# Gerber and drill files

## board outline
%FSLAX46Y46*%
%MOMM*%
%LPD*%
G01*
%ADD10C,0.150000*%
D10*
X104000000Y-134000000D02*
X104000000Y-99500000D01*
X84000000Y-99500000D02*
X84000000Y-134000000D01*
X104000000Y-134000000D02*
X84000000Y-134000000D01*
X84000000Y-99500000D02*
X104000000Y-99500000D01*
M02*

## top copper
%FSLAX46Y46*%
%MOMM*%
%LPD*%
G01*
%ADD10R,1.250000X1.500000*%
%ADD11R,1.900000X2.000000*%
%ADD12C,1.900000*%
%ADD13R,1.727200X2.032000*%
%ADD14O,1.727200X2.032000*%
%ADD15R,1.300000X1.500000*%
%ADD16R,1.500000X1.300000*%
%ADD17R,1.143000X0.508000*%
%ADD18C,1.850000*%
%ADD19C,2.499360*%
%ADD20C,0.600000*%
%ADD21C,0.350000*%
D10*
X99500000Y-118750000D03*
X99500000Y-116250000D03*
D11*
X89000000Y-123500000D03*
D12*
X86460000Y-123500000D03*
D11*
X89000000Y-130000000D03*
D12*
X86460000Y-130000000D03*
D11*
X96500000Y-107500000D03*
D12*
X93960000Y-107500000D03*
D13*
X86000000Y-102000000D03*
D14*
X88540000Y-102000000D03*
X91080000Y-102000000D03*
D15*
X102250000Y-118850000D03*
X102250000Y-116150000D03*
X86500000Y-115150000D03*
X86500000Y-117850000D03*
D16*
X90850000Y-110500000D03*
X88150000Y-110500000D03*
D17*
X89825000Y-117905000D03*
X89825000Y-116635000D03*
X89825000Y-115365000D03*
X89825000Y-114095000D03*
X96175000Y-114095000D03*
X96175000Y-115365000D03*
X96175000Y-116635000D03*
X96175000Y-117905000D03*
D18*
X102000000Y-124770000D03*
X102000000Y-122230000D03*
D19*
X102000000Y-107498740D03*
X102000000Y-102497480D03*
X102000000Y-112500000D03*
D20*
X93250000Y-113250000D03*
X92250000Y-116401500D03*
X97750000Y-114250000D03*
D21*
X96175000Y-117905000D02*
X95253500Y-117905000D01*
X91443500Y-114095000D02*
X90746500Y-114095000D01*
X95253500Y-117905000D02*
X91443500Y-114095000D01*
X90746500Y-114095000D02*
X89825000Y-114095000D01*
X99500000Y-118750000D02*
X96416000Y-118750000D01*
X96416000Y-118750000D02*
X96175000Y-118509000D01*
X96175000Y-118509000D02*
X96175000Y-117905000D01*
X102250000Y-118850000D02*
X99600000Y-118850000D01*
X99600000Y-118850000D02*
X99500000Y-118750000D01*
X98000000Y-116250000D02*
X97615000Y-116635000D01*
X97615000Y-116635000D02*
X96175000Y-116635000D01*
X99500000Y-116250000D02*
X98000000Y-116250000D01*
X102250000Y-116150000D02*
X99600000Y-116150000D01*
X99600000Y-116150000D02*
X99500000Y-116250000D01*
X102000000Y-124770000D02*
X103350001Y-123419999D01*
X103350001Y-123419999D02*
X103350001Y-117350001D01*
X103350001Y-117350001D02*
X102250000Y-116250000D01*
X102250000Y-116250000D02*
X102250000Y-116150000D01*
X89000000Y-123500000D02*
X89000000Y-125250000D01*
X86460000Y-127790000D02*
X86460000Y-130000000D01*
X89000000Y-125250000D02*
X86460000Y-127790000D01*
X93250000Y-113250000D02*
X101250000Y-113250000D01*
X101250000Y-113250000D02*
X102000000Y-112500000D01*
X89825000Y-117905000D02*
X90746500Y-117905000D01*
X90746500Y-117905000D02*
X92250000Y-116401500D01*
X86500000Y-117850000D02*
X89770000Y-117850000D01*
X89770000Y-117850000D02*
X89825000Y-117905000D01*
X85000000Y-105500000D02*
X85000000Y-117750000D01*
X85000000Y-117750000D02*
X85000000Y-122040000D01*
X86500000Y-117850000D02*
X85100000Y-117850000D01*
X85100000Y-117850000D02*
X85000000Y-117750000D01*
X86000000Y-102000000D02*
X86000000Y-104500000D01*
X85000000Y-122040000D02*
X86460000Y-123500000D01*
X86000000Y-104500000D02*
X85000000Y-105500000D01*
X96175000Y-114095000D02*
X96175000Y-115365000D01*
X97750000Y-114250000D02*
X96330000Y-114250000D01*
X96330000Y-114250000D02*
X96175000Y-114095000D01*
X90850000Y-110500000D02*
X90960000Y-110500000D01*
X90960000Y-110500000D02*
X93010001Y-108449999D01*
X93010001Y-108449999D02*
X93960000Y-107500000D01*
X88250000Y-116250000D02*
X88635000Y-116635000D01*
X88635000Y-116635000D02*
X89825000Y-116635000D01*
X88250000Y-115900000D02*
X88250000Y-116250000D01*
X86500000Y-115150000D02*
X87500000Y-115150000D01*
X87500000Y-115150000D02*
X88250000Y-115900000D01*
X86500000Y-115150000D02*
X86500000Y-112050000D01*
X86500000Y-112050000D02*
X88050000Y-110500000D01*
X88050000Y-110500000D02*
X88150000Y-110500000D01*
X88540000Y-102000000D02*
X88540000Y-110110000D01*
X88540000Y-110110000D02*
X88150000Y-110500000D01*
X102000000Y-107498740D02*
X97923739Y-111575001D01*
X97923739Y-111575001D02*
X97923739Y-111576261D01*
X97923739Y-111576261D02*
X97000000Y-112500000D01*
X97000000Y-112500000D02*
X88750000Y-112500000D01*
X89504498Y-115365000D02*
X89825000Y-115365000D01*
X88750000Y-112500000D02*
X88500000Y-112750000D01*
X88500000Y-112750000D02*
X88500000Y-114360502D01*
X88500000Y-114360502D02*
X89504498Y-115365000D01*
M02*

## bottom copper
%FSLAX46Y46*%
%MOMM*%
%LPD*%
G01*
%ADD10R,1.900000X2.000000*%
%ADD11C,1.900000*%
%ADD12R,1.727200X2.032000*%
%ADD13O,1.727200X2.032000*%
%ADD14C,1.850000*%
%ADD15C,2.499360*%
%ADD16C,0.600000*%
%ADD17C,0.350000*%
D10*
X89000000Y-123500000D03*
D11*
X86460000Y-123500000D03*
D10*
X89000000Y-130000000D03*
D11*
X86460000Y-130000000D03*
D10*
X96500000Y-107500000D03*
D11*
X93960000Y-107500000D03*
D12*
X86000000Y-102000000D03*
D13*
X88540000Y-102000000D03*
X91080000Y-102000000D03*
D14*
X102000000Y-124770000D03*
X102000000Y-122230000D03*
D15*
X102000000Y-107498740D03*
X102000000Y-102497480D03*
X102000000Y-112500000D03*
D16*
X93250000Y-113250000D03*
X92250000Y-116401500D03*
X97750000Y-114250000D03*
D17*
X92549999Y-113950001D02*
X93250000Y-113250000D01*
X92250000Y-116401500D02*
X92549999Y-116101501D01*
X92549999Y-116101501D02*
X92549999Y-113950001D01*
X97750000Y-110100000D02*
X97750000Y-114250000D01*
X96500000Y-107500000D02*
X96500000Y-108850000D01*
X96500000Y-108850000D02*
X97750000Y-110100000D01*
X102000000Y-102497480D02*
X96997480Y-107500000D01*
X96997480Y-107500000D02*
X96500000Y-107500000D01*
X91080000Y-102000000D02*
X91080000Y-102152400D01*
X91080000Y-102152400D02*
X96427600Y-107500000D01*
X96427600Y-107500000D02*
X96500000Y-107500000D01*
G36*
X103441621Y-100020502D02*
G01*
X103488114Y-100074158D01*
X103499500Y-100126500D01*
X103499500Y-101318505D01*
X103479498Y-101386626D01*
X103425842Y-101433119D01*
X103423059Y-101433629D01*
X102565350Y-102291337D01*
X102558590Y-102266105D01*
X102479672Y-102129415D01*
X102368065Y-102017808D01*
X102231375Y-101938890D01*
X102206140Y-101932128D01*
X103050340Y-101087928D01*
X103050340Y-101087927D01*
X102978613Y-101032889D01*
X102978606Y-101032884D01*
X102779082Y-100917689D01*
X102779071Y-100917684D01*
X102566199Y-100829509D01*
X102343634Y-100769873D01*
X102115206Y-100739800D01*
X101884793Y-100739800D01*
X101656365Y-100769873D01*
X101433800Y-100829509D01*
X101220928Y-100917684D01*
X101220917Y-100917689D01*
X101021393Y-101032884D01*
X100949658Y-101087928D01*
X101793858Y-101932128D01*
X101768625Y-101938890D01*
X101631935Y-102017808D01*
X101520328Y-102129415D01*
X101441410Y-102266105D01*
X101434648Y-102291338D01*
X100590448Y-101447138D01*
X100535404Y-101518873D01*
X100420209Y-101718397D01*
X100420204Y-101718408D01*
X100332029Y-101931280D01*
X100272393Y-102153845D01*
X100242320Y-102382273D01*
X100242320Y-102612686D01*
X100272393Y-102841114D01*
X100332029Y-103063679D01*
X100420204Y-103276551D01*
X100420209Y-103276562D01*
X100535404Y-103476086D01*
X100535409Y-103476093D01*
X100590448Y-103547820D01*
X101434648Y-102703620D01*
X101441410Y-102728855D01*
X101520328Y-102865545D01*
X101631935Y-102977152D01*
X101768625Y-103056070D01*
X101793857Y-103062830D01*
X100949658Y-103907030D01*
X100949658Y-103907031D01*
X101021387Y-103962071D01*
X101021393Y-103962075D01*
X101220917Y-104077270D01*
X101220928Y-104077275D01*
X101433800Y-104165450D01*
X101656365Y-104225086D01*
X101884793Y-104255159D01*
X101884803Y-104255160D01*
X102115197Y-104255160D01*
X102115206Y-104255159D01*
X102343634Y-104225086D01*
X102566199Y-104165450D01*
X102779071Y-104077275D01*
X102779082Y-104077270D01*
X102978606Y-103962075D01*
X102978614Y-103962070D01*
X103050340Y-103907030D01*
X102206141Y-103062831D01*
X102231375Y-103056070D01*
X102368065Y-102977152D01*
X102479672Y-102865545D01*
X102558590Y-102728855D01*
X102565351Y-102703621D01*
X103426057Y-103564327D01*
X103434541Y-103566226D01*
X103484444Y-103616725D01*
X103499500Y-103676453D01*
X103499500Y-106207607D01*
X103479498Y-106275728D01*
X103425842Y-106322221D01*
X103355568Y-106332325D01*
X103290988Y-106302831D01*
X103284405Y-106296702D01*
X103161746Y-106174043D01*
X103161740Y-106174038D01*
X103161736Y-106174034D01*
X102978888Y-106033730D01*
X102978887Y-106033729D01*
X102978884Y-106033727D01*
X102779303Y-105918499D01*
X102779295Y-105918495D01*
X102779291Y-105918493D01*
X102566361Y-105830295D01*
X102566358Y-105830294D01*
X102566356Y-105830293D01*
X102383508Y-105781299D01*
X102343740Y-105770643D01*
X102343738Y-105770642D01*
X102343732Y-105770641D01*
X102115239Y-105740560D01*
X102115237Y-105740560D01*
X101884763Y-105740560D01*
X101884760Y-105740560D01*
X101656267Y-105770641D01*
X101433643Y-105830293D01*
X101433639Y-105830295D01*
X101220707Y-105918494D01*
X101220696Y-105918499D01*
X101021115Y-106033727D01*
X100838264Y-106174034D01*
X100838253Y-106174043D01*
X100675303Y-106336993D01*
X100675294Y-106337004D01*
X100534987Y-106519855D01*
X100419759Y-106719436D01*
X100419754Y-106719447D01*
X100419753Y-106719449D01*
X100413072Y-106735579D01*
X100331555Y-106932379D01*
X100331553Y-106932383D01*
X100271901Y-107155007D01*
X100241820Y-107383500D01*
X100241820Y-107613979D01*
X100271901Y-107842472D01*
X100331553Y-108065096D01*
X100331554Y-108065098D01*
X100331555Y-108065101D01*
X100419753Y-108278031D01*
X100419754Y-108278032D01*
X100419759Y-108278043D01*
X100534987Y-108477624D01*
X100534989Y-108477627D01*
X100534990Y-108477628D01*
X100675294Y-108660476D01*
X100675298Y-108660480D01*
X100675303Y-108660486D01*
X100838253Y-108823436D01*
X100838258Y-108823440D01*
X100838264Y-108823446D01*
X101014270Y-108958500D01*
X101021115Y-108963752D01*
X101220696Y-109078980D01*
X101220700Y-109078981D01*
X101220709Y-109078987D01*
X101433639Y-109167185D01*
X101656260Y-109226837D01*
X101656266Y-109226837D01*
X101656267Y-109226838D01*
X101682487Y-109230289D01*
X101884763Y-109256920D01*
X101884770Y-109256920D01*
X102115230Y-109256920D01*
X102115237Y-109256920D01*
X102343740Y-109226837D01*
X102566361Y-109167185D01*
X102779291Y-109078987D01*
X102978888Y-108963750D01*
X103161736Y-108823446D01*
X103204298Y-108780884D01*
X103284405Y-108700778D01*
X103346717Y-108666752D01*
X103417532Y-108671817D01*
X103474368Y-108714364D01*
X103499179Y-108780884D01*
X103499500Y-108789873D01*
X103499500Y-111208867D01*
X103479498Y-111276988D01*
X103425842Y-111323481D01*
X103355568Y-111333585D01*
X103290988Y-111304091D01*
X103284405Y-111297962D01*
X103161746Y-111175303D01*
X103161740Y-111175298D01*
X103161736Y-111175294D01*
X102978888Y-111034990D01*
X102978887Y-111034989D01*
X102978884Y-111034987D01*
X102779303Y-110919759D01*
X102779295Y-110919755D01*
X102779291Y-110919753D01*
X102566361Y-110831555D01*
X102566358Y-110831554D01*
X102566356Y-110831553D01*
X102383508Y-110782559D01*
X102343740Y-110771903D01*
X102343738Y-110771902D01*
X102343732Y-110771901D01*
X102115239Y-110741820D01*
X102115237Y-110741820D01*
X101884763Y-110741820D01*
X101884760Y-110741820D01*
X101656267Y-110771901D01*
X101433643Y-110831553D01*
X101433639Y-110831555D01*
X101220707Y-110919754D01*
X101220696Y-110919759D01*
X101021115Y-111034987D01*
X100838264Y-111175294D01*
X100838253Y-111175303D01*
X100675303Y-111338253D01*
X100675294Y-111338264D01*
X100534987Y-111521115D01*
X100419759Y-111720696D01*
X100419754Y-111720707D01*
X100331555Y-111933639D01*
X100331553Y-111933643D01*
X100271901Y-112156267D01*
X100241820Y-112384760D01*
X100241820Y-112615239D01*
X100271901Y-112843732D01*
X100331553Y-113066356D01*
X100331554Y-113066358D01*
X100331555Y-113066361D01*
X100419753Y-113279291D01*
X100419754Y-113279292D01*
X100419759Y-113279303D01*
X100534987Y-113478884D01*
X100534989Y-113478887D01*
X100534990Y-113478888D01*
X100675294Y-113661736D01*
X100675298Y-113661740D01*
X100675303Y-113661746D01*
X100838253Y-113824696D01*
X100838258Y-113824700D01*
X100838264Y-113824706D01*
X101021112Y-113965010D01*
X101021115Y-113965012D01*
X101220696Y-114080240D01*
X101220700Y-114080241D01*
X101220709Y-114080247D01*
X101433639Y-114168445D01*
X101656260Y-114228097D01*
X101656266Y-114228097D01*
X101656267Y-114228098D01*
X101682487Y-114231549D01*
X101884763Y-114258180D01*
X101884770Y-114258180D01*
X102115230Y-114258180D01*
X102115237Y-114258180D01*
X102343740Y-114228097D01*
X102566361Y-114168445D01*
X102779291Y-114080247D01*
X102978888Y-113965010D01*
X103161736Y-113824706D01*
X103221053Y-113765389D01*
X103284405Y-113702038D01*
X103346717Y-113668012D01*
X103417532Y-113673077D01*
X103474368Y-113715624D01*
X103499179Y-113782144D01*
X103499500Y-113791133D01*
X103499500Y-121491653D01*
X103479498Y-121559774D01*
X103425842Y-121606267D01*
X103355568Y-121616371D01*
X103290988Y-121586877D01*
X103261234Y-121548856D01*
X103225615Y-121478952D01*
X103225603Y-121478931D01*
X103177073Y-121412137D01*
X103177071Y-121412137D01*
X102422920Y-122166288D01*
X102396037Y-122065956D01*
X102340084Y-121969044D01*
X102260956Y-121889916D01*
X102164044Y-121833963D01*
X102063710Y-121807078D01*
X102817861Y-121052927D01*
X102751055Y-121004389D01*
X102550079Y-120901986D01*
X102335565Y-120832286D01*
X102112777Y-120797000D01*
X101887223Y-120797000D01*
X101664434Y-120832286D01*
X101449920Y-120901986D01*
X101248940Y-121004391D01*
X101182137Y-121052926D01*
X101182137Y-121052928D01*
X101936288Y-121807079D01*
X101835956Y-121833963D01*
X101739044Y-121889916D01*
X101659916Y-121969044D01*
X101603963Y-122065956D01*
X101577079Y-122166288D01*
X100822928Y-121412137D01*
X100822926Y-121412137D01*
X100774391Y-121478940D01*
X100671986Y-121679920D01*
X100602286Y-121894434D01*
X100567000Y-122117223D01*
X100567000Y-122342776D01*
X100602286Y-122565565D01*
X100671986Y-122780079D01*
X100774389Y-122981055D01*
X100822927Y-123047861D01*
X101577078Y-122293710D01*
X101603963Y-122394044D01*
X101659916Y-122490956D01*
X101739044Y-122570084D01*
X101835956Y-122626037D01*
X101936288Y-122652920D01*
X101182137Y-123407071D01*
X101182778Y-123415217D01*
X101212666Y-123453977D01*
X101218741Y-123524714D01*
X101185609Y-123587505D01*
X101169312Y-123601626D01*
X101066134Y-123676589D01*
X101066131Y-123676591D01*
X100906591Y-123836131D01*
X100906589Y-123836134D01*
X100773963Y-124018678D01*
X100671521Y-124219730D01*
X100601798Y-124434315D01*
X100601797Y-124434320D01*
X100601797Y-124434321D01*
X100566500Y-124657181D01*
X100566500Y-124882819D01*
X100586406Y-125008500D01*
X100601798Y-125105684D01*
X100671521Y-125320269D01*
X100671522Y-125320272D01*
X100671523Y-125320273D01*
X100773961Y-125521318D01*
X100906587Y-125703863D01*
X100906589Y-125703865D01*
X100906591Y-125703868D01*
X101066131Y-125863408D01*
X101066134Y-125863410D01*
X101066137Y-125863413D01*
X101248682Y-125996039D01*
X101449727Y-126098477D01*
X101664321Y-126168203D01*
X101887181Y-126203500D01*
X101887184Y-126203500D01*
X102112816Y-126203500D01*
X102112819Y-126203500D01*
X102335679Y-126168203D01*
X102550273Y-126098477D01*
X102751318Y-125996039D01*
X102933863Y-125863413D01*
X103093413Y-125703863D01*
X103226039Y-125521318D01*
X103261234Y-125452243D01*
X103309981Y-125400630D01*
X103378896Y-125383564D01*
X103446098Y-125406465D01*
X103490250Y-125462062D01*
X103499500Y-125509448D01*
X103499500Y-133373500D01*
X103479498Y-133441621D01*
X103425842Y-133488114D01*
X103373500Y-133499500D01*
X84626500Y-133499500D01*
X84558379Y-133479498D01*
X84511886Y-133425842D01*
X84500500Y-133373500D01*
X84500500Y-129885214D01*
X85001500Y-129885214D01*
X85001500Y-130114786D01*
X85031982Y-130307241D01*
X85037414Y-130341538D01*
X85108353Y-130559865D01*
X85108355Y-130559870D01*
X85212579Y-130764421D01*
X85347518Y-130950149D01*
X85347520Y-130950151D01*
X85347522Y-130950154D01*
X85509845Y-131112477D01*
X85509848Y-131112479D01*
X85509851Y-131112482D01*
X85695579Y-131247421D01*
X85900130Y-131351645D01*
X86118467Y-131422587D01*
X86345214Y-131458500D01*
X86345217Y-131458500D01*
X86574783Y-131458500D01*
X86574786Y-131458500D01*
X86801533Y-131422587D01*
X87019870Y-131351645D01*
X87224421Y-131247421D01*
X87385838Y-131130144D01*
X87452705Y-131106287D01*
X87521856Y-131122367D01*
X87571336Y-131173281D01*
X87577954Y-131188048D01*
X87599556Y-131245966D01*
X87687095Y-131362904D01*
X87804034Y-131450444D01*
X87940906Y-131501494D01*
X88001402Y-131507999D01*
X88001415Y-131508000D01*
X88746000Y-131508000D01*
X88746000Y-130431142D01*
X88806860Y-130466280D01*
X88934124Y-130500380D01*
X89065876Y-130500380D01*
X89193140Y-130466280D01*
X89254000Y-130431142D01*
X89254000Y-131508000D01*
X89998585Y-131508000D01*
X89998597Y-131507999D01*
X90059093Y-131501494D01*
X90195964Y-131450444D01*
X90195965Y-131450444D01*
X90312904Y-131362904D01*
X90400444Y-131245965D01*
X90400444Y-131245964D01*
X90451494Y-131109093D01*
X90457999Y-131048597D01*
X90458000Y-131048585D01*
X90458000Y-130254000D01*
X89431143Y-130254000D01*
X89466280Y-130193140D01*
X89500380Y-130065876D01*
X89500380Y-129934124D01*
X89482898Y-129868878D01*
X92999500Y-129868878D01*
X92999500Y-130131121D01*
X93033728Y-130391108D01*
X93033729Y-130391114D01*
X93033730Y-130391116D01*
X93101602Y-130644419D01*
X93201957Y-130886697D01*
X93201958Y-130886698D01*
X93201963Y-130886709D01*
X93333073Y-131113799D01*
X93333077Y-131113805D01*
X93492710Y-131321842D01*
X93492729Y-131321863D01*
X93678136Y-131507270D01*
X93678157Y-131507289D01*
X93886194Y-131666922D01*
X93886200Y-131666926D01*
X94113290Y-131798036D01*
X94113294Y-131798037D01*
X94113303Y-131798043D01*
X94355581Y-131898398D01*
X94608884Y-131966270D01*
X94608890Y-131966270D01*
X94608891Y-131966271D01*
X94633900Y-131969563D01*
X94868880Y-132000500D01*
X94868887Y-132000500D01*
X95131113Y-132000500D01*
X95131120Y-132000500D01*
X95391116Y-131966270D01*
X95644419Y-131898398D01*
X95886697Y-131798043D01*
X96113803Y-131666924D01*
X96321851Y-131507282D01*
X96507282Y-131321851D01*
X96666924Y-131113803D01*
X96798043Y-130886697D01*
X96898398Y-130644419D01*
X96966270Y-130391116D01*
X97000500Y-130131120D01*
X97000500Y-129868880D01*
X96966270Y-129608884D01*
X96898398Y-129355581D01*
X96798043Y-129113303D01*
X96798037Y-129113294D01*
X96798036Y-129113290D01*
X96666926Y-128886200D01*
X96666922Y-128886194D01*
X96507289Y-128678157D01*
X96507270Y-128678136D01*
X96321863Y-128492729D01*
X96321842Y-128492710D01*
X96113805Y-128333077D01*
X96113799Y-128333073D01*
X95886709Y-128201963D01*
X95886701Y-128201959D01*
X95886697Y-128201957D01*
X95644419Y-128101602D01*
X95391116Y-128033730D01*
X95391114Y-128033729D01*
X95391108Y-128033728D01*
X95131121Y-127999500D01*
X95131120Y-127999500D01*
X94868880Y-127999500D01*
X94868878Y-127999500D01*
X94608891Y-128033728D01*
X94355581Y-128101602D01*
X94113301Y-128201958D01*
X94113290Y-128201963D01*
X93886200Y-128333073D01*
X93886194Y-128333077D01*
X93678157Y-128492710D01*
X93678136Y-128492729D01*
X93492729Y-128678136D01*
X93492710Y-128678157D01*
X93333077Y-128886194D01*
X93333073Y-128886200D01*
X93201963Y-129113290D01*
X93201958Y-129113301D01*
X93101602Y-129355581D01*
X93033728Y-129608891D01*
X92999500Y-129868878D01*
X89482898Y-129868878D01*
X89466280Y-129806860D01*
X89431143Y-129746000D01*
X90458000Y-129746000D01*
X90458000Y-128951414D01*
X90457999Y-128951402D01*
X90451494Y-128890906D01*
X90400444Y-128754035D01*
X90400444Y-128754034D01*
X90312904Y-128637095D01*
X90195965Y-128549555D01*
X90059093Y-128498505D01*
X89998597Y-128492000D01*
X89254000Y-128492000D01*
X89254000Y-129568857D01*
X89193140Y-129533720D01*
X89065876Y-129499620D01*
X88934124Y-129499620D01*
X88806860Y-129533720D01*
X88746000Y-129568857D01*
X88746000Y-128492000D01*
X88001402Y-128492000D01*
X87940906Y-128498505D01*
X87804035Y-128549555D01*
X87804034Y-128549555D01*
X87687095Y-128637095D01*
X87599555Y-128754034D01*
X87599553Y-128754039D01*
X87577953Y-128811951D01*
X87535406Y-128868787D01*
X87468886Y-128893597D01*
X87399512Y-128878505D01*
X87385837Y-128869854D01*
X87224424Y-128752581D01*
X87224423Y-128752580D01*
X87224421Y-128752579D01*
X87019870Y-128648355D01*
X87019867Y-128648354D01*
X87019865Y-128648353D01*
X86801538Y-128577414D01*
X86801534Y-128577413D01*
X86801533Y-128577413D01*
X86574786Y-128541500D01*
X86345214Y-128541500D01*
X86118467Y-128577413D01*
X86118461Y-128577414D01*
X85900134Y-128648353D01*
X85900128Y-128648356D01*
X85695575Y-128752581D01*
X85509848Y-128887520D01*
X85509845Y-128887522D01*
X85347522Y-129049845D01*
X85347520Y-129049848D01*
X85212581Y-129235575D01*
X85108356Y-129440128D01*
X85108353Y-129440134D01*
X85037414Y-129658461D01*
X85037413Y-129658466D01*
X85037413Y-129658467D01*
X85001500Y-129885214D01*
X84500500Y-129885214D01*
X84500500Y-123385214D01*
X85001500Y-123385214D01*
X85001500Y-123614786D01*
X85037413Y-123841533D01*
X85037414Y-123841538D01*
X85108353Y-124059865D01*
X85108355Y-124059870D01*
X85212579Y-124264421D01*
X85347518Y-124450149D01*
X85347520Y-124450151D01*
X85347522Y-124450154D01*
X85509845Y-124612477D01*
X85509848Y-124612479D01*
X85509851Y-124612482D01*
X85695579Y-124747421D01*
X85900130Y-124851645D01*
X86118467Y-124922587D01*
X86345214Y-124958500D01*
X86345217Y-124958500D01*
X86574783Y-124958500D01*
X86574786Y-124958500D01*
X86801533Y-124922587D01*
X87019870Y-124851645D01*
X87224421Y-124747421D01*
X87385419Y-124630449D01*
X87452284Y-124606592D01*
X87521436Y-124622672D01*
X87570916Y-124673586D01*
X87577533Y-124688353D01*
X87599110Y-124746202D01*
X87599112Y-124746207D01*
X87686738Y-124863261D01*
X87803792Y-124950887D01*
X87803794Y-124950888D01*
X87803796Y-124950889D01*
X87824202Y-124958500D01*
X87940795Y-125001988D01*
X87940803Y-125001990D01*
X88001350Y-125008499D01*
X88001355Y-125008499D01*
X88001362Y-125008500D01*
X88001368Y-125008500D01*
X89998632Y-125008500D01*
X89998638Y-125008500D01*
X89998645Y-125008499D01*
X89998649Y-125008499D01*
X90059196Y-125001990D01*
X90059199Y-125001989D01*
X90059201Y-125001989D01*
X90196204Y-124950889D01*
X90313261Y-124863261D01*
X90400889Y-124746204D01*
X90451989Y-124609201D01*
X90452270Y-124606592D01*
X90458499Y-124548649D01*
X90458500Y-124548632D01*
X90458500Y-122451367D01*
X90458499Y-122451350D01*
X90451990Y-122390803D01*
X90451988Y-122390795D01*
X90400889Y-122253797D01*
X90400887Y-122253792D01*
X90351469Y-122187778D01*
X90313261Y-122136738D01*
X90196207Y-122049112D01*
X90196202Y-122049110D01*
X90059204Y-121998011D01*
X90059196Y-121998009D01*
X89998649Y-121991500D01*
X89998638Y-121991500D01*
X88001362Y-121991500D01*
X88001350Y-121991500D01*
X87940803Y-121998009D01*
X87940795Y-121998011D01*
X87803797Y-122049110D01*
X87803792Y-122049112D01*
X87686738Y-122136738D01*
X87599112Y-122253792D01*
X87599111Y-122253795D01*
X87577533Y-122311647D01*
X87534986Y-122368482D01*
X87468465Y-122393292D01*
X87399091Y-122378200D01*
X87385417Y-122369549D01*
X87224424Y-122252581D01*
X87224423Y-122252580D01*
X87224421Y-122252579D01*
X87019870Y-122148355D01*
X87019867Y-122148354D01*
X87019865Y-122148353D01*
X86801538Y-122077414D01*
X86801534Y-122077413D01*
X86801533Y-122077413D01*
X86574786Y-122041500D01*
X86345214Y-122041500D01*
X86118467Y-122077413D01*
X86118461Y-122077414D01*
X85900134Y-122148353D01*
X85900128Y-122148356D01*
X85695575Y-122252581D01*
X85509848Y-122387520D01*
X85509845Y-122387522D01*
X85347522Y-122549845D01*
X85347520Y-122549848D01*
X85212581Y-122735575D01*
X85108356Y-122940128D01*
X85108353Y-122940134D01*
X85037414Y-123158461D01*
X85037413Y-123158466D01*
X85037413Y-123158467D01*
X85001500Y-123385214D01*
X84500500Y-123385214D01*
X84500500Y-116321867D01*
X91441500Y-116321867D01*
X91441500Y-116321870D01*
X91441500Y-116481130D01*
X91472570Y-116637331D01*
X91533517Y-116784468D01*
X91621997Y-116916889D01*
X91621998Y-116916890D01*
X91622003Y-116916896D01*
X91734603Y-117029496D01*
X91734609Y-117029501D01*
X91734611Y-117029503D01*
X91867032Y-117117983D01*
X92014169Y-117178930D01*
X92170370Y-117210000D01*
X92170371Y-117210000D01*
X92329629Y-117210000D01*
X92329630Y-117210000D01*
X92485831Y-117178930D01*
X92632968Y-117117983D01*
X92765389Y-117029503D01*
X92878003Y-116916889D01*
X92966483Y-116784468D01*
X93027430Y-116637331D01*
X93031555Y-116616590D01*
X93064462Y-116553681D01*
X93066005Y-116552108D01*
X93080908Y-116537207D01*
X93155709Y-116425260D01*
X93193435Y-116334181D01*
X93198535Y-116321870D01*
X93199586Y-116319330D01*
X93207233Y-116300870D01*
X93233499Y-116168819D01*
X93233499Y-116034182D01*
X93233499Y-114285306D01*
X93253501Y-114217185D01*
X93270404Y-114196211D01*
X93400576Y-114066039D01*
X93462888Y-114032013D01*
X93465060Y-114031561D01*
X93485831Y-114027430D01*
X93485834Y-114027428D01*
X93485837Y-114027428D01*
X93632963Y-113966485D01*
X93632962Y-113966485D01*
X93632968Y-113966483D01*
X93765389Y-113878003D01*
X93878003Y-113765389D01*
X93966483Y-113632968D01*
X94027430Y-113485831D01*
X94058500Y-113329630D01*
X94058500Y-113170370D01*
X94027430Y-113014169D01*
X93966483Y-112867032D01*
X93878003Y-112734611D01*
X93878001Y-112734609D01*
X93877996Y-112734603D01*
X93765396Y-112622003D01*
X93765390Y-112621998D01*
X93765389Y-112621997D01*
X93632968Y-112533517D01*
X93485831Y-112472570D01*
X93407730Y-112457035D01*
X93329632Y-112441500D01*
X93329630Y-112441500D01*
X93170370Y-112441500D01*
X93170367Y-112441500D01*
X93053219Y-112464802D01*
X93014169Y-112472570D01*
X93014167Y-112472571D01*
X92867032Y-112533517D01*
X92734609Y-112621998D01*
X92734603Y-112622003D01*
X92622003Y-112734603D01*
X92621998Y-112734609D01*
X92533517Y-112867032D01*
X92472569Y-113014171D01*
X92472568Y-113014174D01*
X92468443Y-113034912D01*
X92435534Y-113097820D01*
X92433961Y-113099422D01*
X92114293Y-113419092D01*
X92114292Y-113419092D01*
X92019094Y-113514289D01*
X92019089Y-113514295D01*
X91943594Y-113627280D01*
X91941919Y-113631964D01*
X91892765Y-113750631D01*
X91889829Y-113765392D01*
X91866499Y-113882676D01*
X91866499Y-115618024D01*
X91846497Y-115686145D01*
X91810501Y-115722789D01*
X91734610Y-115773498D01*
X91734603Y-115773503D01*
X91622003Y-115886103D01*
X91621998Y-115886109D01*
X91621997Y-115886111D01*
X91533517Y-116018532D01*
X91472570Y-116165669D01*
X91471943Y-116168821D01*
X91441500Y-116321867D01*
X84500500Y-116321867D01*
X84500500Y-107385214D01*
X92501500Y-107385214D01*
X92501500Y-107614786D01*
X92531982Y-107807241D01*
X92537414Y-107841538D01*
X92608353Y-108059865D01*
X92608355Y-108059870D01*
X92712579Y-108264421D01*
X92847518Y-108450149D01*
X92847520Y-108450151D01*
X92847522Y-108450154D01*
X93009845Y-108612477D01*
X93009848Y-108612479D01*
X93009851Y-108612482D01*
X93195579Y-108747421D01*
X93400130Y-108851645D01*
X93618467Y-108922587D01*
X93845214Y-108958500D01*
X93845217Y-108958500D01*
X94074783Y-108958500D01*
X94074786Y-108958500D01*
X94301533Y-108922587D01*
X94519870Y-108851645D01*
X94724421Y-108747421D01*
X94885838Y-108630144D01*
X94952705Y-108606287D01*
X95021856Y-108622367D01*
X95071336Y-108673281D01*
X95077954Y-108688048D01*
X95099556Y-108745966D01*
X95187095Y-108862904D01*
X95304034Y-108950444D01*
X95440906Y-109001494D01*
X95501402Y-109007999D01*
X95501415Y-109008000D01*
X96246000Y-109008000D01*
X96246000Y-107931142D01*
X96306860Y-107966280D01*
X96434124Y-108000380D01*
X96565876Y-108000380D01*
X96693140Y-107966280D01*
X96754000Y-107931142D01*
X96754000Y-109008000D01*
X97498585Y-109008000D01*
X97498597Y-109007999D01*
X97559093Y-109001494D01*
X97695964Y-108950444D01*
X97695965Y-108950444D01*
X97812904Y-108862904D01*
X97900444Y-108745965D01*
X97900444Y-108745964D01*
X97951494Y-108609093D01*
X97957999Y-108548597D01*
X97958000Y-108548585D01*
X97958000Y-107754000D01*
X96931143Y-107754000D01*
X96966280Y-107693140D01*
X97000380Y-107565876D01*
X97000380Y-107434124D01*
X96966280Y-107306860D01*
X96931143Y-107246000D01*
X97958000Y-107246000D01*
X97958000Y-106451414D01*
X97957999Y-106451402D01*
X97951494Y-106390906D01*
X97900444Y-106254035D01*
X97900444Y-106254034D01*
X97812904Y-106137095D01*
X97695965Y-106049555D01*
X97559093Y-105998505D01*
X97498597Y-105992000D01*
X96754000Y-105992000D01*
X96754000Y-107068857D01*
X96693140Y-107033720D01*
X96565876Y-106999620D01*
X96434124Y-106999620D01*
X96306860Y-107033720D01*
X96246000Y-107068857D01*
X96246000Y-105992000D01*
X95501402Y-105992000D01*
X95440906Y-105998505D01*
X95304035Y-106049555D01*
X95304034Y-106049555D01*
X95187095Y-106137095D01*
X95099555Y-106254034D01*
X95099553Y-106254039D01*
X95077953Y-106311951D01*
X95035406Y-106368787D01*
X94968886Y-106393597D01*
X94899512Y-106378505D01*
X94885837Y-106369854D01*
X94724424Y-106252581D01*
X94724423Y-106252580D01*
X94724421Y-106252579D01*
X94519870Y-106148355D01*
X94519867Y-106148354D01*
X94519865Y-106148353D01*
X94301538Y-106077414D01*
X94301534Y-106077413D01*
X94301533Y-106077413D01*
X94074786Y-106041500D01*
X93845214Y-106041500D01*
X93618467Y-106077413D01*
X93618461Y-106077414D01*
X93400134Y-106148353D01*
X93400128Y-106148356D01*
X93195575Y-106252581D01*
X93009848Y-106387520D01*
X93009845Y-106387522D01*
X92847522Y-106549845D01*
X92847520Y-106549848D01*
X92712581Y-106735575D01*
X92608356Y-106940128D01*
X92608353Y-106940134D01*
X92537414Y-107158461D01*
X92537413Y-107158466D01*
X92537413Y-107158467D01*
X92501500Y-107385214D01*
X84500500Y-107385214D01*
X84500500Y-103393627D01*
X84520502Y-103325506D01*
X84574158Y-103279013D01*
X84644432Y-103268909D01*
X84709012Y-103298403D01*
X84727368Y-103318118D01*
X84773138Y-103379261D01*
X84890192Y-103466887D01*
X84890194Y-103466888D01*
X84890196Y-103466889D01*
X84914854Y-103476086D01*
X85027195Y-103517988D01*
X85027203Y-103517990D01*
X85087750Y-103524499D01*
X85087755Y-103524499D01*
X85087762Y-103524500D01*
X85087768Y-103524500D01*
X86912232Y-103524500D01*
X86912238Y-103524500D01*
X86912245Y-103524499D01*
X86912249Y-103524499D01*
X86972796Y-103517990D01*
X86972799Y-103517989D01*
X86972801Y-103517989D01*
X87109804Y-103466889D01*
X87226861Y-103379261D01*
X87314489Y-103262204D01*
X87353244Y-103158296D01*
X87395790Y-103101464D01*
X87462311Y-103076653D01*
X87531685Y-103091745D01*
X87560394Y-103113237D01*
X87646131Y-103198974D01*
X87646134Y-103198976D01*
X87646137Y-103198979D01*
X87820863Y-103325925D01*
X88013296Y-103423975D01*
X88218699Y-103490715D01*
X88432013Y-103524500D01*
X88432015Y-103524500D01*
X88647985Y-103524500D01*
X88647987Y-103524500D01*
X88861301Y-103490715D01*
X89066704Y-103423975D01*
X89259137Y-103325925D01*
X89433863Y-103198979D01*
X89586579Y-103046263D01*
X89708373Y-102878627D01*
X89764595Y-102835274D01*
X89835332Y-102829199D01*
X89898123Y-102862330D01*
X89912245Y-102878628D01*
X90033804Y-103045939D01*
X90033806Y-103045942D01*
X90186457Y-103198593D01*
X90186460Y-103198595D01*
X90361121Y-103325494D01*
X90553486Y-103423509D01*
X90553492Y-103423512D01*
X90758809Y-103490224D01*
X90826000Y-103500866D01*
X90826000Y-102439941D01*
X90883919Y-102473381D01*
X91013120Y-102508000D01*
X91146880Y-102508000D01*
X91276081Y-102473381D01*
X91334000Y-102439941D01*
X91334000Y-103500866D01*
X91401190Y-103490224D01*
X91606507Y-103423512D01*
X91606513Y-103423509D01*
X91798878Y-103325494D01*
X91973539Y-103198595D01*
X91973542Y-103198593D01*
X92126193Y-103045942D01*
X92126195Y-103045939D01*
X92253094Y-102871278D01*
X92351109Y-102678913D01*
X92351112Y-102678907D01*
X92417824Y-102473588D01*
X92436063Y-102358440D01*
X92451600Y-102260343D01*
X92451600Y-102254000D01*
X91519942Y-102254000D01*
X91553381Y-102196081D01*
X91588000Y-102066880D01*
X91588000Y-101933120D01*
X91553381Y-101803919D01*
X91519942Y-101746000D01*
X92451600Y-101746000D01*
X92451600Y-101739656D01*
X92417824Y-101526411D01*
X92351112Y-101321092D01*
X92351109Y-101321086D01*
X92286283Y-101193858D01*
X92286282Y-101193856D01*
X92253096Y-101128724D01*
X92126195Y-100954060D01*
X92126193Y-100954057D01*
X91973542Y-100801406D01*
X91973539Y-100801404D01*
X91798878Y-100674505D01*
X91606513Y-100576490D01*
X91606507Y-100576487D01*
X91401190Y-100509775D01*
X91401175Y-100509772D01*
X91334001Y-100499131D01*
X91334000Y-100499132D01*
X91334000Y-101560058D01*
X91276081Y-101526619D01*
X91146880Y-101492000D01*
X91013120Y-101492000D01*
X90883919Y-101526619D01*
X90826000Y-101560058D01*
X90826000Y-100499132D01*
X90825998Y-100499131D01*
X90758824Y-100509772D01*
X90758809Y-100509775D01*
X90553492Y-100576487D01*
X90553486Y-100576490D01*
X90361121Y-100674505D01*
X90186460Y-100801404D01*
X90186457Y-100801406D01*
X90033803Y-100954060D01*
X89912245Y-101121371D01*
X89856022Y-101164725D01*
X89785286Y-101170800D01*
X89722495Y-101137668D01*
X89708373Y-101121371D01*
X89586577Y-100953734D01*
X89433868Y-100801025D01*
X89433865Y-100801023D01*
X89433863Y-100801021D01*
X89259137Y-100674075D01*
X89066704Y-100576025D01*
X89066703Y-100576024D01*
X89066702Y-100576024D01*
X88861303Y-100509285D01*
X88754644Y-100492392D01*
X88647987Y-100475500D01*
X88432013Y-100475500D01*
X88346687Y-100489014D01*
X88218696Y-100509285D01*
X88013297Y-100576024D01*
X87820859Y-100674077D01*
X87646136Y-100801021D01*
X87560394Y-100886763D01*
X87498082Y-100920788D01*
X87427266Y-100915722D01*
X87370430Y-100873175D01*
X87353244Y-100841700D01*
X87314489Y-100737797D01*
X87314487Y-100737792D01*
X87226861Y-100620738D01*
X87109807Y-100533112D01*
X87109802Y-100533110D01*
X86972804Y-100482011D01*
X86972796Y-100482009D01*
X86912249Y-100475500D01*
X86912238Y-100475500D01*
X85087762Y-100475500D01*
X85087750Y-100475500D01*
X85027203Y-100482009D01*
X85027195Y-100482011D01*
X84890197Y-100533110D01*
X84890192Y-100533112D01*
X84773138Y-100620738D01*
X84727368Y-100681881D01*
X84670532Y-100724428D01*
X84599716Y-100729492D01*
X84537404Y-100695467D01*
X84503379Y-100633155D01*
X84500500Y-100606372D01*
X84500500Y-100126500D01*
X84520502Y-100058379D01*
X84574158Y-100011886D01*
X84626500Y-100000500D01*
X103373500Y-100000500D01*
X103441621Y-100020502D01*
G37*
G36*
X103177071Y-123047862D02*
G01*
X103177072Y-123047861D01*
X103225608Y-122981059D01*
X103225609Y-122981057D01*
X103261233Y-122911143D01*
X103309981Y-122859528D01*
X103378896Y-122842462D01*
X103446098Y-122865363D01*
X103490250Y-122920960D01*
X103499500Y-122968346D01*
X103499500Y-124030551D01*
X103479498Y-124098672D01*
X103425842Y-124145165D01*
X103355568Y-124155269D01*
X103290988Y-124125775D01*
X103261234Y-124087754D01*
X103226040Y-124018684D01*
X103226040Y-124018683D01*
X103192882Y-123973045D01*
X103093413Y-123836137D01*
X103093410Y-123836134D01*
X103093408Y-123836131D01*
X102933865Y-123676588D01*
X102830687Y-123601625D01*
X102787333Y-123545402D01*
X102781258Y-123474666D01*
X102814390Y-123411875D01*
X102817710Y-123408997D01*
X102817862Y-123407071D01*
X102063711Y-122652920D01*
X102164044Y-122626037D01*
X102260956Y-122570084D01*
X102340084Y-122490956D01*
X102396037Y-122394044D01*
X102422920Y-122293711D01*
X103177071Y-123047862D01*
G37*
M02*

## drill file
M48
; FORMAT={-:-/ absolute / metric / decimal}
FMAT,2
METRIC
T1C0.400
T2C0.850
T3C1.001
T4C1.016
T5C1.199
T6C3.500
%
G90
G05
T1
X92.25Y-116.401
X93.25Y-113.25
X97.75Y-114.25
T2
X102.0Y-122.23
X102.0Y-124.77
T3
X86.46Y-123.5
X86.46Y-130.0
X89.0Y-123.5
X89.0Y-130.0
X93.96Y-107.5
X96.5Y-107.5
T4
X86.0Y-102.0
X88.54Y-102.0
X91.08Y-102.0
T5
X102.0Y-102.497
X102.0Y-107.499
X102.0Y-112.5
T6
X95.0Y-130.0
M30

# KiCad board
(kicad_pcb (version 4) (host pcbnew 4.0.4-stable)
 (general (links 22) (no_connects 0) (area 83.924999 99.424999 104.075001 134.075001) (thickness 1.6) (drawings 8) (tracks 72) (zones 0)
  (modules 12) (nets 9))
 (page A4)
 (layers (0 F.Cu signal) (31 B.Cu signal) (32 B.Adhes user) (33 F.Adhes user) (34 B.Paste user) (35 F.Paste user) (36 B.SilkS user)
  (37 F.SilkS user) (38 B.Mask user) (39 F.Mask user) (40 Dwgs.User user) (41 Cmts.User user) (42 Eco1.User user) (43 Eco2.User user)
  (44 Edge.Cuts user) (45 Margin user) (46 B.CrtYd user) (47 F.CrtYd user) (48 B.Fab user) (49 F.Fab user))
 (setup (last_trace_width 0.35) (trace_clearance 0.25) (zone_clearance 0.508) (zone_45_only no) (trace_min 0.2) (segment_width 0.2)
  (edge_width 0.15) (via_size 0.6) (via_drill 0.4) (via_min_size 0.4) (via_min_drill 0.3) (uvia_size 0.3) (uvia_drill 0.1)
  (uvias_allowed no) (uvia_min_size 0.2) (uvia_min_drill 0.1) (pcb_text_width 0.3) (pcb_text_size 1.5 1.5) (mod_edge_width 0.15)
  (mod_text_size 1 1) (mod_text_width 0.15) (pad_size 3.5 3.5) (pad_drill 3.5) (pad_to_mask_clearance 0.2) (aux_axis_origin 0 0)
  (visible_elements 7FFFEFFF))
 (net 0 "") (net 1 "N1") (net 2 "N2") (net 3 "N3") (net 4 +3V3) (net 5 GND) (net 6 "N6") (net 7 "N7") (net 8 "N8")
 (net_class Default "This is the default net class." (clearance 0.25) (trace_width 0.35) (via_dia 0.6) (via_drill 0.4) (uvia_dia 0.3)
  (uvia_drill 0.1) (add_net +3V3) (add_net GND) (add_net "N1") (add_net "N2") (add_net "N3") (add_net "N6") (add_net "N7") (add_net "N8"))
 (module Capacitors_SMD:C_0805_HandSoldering (layer F.Cu) (at 99.5 117.5 90)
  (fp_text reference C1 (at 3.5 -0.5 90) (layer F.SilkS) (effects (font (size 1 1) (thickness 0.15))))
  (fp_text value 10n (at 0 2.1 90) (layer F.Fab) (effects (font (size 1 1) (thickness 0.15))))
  (pad 1 smd rect (at -1.25 0 90) (size 1.5 1.25) (layers F.Cu F.Paste F.Mask) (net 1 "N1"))
  (pad 2 smd rect (at 1.25 0 90) (size 1.5 1.25) (layers F.Cu F.Paste F.Mask) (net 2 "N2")))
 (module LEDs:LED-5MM (layer B.Cu) (at 89 123.5 180)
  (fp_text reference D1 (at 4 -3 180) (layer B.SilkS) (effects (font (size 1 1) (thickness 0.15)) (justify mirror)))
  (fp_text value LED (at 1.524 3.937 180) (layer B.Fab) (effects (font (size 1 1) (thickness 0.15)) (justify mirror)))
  (pad 1 thru_hole rect (at 0 0 90) (size 2 1.9) (drill 1.00076) (layers *.Cu *.Mask B.SilkS) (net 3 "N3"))
  (pad 2 thru_hole circle (at 2.54 0 180) (size 1.9 1.9) (drill 1.00076) (layers *.Cu *.Mask B.SilkS) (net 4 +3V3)))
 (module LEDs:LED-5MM (layer B.Cu) (at 89 130 180)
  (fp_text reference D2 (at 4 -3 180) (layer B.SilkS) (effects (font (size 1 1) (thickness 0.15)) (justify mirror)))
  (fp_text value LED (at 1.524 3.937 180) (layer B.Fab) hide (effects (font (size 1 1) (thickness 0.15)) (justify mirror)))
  (pad 1 thru_hole rect (at 0 0 90) (size 2 1.9) (drill 1.00076) (layers *.Cu *.Mask B.SilkS) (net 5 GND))
  (pad 2 thru_hole circle (at 2.54 0 180) (size 1.9 1.9) (drill 1.00076) (layers *.Cu *.Mask B.SilkS) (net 3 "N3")))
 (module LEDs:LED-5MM (layer B.Cu) (at 96.5 107.5 180)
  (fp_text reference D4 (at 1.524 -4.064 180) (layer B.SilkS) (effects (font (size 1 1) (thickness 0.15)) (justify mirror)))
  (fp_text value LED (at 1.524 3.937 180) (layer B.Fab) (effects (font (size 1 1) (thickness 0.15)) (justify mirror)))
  (pad 1 thru_hole rect (at 0 0 90) (size 2 1.9) (drill 1.00076) (layers *.Cu *.Mask B.SilkS) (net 5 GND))
  (pad 2 thru_hole circle (at 2.54 0 180) (size 1.9 1.9) (drill 1.00076) (layers *.Cu *.Mask B.SilkS) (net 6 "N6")))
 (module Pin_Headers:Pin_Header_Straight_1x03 (layer F.Cu) (at 86 102 90)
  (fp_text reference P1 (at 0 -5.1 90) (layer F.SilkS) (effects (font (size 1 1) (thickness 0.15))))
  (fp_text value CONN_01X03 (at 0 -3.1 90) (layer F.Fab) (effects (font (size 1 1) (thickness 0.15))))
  (pad 1 thru_hole rect (at 0 0 90) (size 2.032 1.7272) (drill 1.016) (layers *.Cu *.Mask F.SilkS) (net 4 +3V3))
  (pad 2 thru_hole oval (at 0 2.54 90) (size 2.032 1.7272) (drill 1.016) (layers *.Cu *.Mask F.SilkS) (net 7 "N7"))
  (pad 3 thru_hole oval (at 0 5.08 90) (size 2.032 1.7272) (drill 1.016) (layers *.Cu *.Mask F.SilkS) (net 5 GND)))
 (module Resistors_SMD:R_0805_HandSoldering (layer F.Cu) (at 102.25 117.5 90)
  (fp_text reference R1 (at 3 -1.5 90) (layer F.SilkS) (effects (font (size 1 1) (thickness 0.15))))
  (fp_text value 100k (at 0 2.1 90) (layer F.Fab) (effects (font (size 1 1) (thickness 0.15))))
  (pad 1 smd rect (at -1.35 0 90) (size 1.5 1.3) (layers F.Cu F.Paste F.Mask) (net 1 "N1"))
  (pad 2 smd rect (at 1.35 0 90) (size 1.5 1.3) (layers F.Cu F.Paste F.Mask) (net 2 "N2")))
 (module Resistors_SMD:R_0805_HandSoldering (layer F.Cu) (at 86.5 116.5 270)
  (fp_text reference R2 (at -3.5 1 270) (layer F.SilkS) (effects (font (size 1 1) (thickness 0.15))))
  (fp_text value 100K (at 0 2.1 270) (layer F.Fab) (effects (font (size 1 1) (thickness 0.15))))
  (pad 1 smd rect (at -1.35 0 270) (size 1.5 1.3) (layers F.Cu F.Paste F.Mask) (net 7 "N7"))
  (pad 2 smd rect (at 1.35 0 270) (size 1.5 1.3) (layers F.Cu F.Paste F.Mask) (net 4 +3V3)))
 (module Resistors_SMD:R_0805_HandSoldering (layer F.Cu) (at 89.5 110.5 180)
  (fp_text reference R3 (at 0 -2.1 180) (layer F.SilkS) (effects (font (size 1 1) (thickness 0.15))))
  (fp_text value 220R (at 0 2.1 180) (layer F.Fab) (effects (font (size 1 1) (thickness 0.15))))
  (pad 1 smd rect (at -1.35 0 180) (size 1.5 1.3) (layers F.Cu F.Paste F.Mask) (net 6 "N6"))
  (pad 2 smd rect (at 1.35 0 180) (size 1.5 1.3) (layers F.Cu F.Paste F.Mask) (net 7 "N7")))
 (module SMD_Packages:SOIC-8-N (layer F.Cu) (at 93 116 90)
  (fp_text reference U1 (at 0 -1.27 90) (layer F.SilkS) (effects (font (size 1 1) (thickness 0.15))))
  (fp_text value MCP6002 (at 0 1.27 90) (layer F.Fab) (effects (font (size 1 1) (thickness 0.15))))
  (pad 8 smd rect (at -1.905 -3.175 90) (size 0.508 1.143) (layers F.Cu F.Paste F.Mask) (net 4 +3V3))
  (pad 7 smd rect (at -0.635 -3.175 90) (size 0.508 1.143) (layers F.Cu F.Paste F.Mask) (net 7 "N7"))
  (pad 6 smd rect (at 0.635 -3.175 90) (size 0.508 1.143) (layers F.Cu F.Paste F.Mask) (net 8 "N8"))
  (pad 5 smd rect (at 1.905 -3.175 90) (size 0.508 1.143) (layers F.Cu F.Paste F.Mask) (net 1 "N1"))
  (pad 4 smd rect (at 1.905 3.175 90) (size 0.508 1.143) (layers F.Cu F.Paste F.Mask) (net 5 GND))
  (pad 3 smd rect (at 0.635 3.175 90) (size 0.508 1.143) (layers F.Cu F.Paste F.Mask) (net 5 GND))
  (pad 2 smd rect (at -0.635 3.175 90) (size 0.508 1.143) (layers F.Cu F.Paste F.Mask) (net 2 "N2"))
  (pad 1 smd rect (at -1.905 3.175 90) (size 0.508 1.143) (layers F.Cu F.Paste F.Mask) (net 1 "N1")))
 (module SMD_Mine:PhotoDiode (layer B.Cu) (at 102 123.5)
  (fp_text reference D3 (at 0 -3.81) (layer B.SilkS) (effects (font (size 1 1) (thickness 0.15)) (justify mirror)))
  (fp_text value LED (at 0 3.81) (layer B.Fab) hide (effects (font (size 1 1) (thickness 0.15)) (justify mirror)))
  (pad 1 thru_hole circle (at 0 1.27) (size 1.85 1.85) (drill 0.85) (layers *.Cu *.Mask) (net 2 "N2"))
  (pad 2 thru_hole circle (at 0 -1.27) (size 1.85 1.85) (drill 0.85) (layers *.Cu *.Mask) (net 5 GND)))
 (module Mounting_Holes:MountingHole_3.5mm (layer F.Cu) (at 95 130)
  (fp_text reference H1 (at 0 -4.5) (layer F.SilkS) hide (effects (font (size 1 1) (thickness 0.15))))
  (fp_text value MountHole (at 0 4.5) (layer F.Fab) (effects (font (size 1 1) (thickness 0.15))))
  (pad "" np_thru_hole circle (at 0 0) (size 3.5 3.5) (drill 3.5) (layers *.Cu *.Mask F.SilkS)))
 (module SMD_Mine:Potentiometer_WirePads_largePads (layer B.Cu) (at 102 112.5)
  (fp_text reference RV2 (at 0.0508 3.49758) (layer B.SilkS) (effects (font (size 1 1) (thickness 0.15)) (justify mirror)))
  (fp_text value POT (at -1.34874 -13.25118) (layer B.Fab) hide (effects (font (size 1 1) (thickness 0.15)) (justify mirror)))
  (pad 2 thru_hole circle (at 0 -5.00126) (size 2.49936 2.49936) (drill 1.19888) (layers *.Cu *.Mask B.SilkS) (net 8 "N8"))
  (pad 3 thru_hole circle (at 0 -10.00252) (size 2.49936 2.49936) (drill 1.19888) (layers *.Cu *.Mask B.SilkS) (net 5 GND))
  (pad 1 thru_hole circle (at 0 0) (size 2.49936 2.49936) (drill 1.19888) (layers *.Cu *.Mask B.SilkS) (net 4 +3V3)))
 (gr_line (start 104 134) (end 104 99.5) (angle 90) (layer Edge.Cuts) (width 0.15))
 (gr_line (start 84 99.5) (end 84 134) (angle 90) (layer Edge.Cuts) (width 0.15))
 (gr_line (start 104 134) (end 84 134) (angle 90) (layer Edge.Cuts) (width 0.15))
 (gr_line (start 84 99.5) (end 104 99.5) (angle 90) (layer Edge.Cuts) (width 0.15))
 (segment (start 96.175 117.905) (end 95.2535 117.905) (width 0.35) (layer F.Cu) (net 1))
 (segment (start 91.4435 114.095) (end 90.7465 114.095) (width 0.35) (layer F.Cu) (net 1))
 (segment (start 95.2535 117.905) (end 91.4435 114.095) (width 0.35) (layer F.Cu) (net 1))
 (segment (start 90.7465 114.095) (end 89.825 114.095) (width 0.35) (layer F.Cu) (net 1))
 (segment (start 99.5 118.75) (end 96.416 118.75) (width 0.35) (layer F.Cu) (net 1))
 (segment (start 96.416 118.75) (end 96.175 118.509) (width 0.35) (layer F.Cu) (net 1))
 (segment (start 96.175 118.509) (end 96.175 117.905) (width 0.35) (layer F.Cu) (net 1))
 (segment (start 102.25 118.85) (end 99.6 118.85) (width 0.35) (layer F.Cu) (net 1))
 (segment (start 99.6 118.85) (end 99.5 118.75) (width 0.35) (layer F.Cu) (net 1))
 (segment (start 98 116.25) (end 97.615 116.635) (width 0.35) (layer F.Cu) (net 2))
 (segment (start 97.615 116.635) (end 96.175 116.635) (width 0.35) (layer F.Cu) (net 2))
 (segment (start 99.5 116.25) (end 98 116.25) (width 0.35) (layer F.Cu) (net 2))
 (segment (start 102.25 116.15) (end 99.6 116.15) (width 0.35) (layer F.Cu) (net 2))
 (segment (start 99.6 116.15) (end 99.5 116.25) (width 0.35) (layer F.Cu) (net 2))
 (segment (start 102 124.77) (end 103.350001 123.419999) (width 0.35) (layer F.Cu) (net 2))
 (segment (start 103.350001 123.419999) (end 103.350001 117.350001) (width 0.35) (layer F.Cu) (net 2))
 (segment (start 103.350001 117.350001) (end 102.25 116.25) (width 0.35) (layer F.Cu) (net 2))
 (segment (start 102.25 116.25) (end 102.25 116.15) (width 0.35) (layer F.Cu) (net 2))
 (segment (start 89 123.5) (end 89 125.25) (width 0.35) (layer F.Cu) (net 3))
 (segment (start 86.46 127.79) (end 86.46 130) (width 0.35) (layer F.Cu) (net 3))
 (segment (start 89 125.25) (end 86.46 127.79) (width 0.35) (layer F.Cu) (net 3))
 (segment (start 93.25 113.25) (end 101.25 113.25) (width 0.35) (layer F.Cu) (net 4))
 (segment (start 101.25 113.25) (end 102 112.5) (width 0.35) (layer F.Cu) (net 4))
 (segment (start 92.549999 113.950001) (end 93.25 113.25) (width 0.35) (layer B.Cu) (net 4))
 (via (at 93.25 113.25) (size 0.6) (drill 0.4) (layers F.Cu B.Cu) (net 4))
 (segment (start 92.25 116.4015) (end 92.549999 116.101501) (width 0.35) (layer B.Cu) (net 4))
 (segment (start 92.549999 116.101501) (end 92.549999 113.950001) (width 0.35) (layer B.Cu) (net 4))
 (via (at 92.25 116.4015) (size 0.6) (drill 0.4) (layers F.Cu B.Cu) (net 4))
 (segment (start 89.825 117.905) (end 90.7465 117.905) (width 0.35) (layer F.Cu) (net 4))
 (segment (start 90.7465 117.905) (end 92.25 116.4015) (width 0.35) (layer F.Cu) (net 4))
 (segment (start 86.5 117.85) (end 89.77 117.85) (width 0.35) (layer F.Cu) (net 4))
 (segment (start 89.77 117.85) (end 89.825 117.905) (width 0.35) (layer F.Cu) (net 4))
 (segment (start 85 105.5) (end 85 117.75) (width 0.35) (layer F.Cu) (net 4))
 (segment (start 85 117.75) (end 85 122.04) (width 0.35) (layer F.Cu) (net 4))
 (segment (start 86.5 117.85) (end 85.1 117.85) (width 0.35) (layer F.Cu) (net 4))
 (segment (start 85.1 117.85) (end 85 117.75) (width 0.35) (layer F.Cu) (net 4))
 (segment (start 86 102) (end 86 104.5) (width 0.35) (layer F.Cu) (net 4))
 (segment (start 85 122.04) (end 86.46 123.5) (width 0.35) (layer F.Cu) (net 4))
 (segment (start 86 104.5) (end 85 105.5) (width 0.35) (layer F.Cu) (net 4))
 (segment (start 96.175 114.095) (end 96.175 115.365) (width 0.35) (layer F.Cu) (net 5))
 (segment (start 97.75 114.25) (end 96.33 114.25) (width 0.35) (layer F.Cu) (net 5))
 (segment (start 96.33 114.25) (end 96.175 114.095) (width 0.35) (layer F.Cu) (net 5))
 (segment (start 97.75 110.1) (end 97.75 114.25) (width 0.35) (layer B.Cu) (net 5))
 (via (at 97.75 114.25) (size 0.6) (drill 0.4) (layers F.Cu B.Cu) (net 5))
 (segment (start 96.5 107.5) (end 96.5 108.85) (width 0.35) (layer B.Cu) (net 5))
 (segment (start 96.5 108.85) (end 97.75 110.1) (width 0.35) (layer B.Cu) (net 5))
 (segment (start 102 102.49748) (end 96.99748 107.5) (width 0.35) (layer B.Cu) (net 5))
 (segment (start 96.99748 107.5) (end 96.5 107.5) (width 0.35) (layer B.Cu) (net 5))
 (segment (start 91.08 102) (end 91.08 102.1524) (width 0.35) (layer B.Cu) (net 5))
 (segment (start 91.08 102.1524) (end 96.4276 107.5) (width 0.35) (layer B.Cu) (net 5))
 (segment (start 96.4276 107.5) (end 96.5 107.5) (width 0.35) (layer B.Cu) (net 5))
 (segment (start 90.85 110.5) (end 90.96 110.5) (width 0.35) (layer F.Cu) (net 6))
 (segment (start 90.96 110.5) (end 93.010001 108.449999) (width 0.35) (layer F.Cu) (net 6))
 (segment (start 93.010001 108.449999) (end 93.96 107.5) (width 0.35) (layer F.Cu) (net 6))
 (segment (start 88.25 116.25) (end 88.635 116.635) (width 0.35) (layer F.Cu) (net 7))
 (segment (start 88.635 116.635) (end 89.825 116.635) (width 0.35) (layer F.Cu) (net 7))
 (segment (start 88.25 115.9) (end 88.25 116.25) (width 0.35) (layer F.Cu) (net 7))
 (segment (start 86.5 115.15) (end 87.5 115.15) (width 0.35) (layer F.Cu) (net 7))
 (segment (start 87.5 115.15) (end 88.25 115.9) (width 0.35) (layer F.Cu) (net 7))
 (segment (start 86.5 115.15) (end 86.5 112.05) (width 0.35) (layer F.Cu) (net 7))
 (segment (start 86.5 112.05) (end 88.05 110.5) (width 0.35) (layer F.Cu) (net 7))
 (segment (start 88.05 110.5) (end 88.15 110.5) (width 0.35) (layer F.Cu) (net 7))
 (segment (start 88.54 102) (end 88.54 110.11) (width 0.35) (layer F.Cu) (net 7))
 (segment (start 88.54 110.11) (end 88.15 110.5) (width 0.35) (layer F.Cu) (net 7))
 (segment (start 102 107.49874) (end 97.923739 111.575001) (width 0.35) (layer F.Cu) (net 8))
 (segment (start 97.923739 111.575001) (end 97.923739 111.576261) (width 0.35) (layer F.Cu) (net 8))
 (segment (start 97.923739 111.576261) (end 97 112.5) (width 0.35) (layer F.Cu) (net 8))
 (segment (start 97 112.5) (end 88.75 112.5) (width 0.35) (layer F.Cu) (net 8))
 (segment (start 89.504498 115.365) (end 89.825 115.365) (width 0.35) (layer F.Cu) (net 8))
 (segment (start 88.75 112.5) (end 88.5 112.75) (width 0.35) (layer F.Cu) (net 8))
 (segment (start 88.5 112.75) (end 88.5 114.360502) (width 0.35) (layer F.Cu) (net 8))
 (segment (start 88.5 114.360502) (end 89.504498 115.365) (width 0.35) (layer F.Cu) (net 8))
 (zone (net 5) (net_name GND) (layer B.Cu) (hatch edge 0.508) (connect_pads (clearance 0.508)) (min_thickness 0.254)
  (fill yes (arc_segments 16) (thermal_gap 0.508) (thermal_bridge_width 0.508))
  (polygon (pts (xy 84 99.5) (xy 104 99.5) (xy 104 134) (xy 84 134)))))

